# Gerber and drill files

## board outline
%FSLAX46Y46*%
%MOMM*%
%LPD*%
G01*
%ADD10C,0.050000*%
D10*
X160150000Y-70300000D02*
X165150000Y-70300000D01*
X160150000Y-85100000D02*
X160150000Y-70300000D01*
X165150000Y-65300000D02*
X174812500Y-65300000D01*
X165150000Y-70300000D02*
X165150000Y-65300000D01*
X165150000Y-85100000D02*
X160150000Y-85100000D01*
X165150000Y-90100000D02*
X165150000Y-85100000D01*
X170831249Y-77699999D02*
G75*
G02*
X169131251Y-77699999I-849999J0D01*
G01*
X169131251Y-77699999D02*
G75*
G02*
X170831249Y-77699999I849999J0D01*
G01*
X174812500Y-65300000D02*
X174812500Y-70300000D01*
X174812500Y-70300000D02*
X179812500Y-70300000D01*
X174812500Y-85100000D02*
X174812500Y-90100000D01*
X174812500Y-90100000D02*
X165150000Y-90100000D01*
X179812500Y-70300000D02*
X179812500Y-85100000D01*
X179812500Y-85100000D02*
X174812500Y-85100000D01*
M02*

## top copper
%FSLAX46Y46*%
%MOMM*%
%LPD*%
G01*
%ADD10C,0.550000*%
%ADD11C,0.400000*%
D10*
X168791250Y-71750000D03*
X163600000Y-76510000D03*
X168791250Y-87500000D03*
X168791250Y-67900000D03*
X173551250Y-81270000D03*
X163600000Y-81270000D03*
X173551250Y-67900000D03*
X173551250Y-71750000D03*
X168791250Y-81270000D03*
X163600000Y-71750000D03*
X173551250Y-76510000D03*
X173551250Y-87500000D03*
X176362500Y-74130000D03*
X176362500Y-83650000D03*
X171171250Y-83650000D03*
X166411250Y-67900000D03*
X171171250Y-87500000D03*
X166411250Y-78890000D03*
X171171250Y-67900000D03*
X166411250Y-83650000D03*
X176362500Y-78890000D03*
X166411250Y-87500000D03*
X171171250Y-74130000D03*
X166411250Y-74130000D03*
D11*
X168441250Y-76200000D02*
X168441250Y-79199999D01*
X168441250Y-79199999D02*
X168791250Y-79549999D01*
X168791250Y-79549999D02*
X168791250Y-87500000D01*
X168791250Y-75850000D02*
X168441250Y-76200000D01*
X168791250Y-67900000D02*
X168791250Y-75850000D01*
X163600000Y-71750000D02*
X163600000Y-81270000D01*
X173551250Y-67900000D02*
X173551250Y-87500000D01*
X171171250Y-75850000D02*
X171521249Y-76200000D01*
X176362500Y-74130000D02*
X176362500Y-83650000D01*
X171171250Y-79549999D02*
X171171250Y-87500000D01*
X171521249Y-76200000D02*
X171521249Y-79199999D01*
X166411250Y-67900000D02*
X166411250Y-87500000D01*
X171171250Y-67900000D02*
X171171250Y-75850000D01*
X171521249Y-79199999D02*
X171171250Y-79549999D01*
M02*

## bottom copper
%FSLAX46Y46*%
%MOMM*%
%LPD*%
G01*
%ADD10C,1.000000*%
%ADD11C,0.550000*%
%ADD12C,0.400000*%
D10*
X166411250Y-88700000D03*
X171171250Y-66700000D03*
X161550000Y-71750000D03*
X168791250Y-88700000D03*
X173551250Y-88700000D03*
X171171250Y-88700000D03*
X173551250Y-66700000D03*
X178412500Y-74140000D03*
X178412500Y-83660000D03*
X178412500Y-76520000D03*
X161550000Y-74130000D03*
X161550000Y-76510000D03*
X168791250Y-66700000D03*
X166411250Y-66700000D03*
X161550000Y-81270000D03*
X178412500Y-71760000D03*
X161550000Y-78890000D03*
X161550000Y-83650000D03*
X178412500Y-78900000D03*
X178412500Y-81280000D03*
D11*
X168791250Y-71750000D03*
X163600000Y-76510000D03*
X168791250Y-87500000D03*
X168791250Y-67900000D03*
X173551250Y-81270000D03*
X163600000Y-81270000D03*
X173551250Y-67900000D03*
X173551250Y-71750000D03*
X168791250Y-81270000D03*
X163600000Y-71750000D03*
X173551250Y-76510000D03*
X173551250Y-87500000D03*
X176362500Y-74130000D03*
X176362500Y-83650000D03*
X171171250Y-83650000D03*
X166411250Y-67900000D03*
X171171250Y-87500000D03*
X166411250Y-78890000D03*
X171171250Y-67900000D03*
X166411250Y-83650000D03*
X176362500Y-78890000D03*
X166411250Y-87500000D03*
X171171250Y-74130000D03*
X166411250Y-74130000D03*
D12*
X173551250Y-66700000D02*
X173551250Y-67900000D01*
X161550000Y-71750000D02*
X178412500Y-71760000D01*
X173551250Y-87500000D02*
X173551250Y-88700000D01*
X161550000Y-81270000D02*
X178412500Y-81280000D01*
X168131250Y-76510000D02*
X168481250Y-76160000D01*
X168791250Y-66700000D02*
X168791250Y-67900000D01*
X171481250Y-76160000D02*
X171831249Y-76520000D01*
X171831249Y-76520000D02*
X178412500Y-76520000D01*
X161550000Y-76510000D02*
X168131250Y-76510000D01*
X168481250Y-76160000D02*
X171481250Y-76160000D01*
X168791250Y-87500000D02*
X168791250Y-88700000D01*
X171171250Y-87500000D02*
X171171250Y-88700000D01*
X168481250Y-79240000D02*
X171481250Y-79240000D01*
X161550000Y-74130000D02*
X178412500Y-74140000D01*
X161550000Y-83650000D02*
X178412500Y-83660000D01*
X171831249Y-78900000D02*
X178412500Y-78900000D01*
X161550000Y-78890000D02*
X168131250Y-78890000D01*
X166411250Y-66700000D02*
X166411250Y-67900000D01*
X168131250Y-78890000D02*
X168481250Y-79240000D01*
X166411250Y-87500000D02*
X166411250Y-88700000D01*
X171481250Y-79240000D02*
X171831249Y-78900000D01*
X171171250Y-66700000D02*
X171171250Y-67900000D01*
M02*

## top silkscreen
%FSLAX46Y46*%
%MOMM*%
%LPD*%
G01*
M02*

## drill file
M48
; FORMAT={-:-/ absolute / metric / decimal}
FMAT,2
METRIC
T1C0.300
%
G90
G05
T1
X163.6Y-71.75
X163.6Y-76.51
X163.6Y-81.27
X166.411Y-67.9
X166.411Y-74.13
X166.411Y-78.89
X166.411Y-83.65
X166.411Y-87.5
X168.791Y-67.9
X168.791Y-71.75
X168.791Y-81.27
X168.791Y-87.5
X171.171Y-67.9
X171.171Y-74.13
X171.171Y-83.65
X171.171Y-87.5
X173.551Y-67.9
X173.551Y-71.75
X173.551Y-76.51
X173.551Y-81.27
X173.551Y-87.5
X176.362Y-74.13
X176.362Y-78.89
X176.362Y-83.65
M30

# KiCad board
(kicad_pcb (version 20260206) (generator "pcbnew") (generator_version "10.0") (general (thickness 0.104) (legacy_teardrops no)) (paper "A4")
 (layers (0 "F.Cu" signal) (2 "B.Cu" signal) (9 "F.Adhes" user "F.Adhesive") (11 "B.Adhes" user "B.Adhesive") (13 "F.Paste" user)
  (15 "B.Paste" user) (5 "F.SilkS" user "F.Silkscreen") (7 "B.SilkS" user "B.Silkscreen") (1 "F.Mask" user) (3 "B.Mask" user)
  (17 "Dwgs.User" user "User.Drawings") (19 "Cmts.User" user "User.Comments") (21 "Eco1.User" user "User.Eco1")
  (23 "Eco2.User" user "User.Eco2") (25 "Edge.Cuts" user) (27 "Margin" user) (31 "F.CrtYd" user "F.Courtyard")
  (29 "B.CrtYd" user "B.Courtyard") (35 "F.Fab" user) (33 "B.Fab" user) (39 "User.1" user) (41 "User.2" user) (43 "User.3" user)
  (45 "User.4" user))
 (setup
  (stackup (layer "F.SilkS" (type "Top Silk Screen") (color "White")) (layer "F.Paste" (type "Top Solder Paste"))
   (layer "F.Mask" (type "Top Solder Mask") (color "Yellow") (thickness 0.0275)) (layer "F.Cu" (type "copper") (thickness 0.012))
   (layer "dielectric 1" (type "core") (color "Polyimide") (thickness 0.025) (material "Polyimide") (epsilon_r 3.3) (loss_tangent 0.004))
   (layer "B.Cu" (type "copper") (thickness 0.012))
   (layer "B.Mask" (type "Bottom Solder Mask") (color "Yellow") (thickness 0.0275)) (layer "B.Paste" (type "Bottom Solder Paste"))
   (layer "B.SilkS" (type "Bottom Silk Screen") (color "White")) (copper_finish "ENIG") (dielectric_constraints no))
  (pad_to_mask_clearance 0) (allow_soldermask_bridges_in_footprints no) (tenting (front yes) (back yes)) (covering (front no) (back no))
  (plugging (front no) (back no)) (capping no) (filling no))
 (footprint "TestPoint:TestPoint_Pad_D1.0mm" (layer "B.Cu") (at 166.41125 88.7)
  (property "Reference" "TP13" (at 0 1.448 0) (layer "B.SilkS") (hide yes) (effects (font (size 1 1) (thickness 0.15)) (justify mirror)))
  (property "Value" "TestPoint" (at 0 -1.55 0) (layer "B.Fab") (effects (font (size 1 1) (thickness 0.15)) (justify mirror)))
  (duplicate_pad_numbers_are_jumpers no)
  (pad "1" smd circle (at 0 0) (size 1 1) (layers "B.Cu" "B.Mask") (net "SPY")))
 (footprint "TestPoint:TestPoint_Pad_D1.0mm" (layer "B.Cu") (at 171.17125 66.7 180)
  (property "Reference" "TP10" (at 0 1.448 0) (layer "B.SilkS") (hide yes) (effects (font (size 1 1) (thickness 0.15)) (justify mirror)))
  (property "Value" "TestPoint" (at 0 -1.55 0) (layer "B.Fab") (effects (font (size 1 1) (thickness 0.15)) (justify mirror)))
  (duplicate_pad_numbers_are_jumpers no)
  (pad "1" smd circle (at 0 0 180) (size 1 1) (layers "B.Cu" "B.Mask") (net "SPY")))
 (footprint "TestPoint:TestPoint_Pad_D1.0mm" (layer "B.Cu") (at 161.55 71.75 -90)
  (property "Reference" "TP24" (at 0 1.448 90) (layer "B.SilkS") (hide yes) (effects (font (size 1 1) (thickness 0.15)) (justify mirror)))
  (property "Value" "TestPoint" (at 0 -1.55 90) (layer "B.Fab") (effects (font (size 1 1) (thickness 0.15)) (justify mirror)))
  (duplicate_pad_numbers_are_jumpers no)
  (pad "1" smd circle (at 0 0 270) (size 1 1) (layers "B.Cu" "B.Mask") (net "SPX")))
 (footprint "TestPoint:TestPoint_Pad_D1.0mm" (layer "B.Cu") (at 168.79125 88.7)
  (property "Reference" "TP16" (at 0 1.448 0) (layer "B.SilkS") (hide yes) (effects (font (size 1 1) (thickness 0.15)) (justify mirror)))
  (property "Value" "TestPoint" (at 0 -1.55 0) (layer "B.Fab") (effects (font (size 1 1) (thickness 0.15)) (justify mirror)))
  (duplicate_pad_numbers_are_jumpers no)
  (pad "1" smd circle (at 0 0) (size 1 1) (layers "B.Cu" "B.Mask") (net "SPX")))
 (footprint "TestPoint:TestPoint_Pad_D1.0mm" (layer "B.Cu") (at 173.55125 88.7)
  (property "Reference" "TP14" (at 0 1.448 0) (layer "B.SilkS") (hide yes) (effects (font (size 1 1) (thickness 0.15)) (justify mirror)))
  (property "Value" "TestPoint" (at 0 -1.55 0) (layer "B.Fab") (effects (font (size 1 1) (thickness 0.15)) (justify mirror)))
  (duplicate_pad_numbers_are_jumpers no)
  (pad "1" smd circle (at 0 0) (size 1 1) (layers "B.Cu" "B.Mask") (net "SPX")))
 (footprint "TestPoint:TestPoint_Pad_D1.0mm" (layer "B.Cu") (at 171.17125 88.7)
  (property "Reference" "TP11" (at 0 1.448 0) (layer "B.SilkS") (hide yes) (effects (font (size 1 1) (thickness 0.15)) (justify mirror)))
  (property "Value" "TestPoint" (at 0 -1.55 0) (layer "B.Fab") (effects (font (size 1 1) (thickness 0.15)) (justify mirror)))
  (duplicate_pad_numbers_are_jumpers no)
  (pad "1" smd circle (at 0 0) (size 1 1) (layers "B.Cu" "B.Mask") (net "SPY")))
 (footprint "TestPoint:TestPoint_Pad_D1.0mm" (layer "B.Cu") (at 173.55125 66.7 180)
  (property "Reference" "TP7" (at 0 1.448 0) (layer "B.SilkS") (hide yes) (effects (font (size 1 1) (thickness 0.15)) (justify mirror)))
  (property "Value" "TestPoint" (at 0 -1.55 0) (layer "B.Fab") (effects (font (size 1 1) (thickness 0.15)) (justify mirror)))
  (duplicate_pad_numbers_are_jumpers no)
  (pad "1" smd circle (at 0 0 180) (size 1 1) (layers "B.Cu" "B.Mask") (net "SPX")))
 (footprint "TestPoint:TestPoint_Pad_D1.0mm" (layer "B.Cu") (at 178.4125 74.14 90)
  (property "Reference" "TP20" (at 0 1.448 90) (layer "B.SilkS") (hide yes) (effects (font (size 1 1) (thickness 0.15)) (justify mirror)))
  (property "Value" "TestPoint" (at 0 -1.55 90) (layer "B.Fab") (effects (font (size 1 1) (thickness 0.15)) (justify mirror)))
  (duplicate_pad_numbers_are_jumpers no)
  (pad "1" smd circle (at 0 0 90) (size 1 1) (layers "B.Cu" "B.Mask") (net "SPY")))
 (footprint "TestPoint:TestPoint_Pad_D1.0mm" (layer "B.Cu") (at 178.4125 83.66 90)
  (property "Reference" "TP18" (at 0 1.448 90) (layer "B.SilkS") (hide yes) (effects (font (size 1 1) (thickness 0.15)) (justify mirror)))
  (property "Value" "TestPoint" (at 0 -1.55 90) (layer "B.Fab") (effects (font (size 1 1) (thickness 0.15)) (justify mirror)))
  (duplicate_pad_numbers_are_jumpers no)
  (pad "1" smd circle (at 0 0 90) (size 1 1) (layers "B.Cu" "B.Mask") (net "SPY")))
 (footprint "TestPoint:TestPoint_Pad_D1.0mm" (layer "B.Cu") (at 178.4125 76.52 90)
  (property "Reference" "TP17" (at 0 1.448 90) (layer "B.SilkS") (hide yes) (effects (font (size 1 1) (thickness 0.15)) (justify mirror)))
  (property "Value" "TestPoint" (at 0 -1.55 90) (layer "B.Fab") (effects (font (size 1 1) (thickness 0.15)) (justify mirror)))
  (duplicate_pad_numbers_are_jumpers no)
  (pad "1" smd circle (at 0 0 90) (size 1 1) (layers "B.Cu" "B.Mask") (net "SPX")))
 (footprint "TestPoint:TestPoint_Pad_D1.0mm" (layer "B.Cu") (at 161.55 74.13 -90)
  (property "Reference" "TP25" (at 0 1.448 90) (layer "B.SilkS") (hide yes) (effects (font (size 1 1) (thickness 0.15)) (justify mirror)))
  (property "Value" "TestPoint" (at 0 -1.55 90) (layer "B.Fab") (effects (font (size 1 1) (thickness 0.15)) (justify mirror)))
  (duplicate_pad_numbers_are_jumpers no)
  (pad "1" smd circle (at 0 0 270) (size 1 1) (layers "B.Cu" "B.Mask") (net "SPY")))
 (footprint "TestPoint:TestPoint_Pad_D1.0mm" (layer "B.Cu") (at 161.55 76.51 -90)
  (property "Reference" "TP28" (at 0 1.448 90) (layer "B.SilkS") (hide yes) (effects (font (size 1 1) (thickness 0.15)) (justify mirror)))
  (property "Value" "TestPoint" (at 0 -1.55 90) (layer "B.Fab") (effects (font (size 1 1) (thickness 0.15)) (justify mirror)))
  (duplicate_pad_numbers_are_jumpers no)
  (pad "1" smd circle (at 0 0 270) (size 1 1) (layers "B.Cu" "B.Mask") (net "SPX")))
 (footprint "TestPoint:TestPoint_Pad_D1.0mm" (layer "B.Cu") (at 168.79125 66.7 180)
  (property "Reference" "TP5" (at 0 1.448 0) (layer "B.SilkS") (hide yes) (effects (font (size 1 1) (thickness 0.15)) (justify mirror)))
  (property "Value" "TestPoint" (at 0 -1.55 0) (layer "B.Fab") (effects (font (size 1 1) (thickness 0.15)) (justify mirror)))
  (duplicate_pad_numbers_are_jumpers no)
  (pad "1" smd circle (at 0 0 180) (size 1 1) (layers "B.Cu" "B.Mask") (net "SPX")))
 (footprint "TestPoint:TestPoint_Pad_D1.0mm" (layer "B.Cu") (at 166.41125 66.7 180)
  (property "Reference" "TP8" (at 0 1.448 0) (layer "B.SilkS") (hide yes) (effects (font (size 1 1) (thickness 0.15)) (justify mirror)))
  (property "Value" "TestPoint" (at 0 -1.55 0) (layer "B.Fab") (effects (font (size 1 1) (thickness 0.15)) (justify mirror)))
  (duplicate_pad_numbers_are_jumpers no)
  (pad "1" smd circle (at 0 0 180) (size 1 1) (layers "B.Cu" "B.Mask") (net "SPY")))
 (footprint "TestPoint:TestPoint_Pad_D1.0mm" (layer "B.Cu") (at 161.55 81.27 -90)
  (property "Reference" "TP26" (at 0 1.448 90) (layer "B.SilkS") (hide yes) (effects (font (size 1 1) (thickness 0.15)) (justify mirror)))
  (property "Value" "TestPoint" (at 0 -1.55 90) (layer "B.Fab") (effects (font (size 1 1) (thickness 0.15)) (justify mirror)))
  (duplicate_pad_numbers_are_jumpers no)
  (pad "1" smd circle (at 0 0 270) (size 1 1) (layers "B.Cu" "B.Mask") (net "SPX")))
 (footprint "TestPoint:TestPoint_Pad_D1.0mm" (layer "B.Cu") (at 178.4125 71.76 90)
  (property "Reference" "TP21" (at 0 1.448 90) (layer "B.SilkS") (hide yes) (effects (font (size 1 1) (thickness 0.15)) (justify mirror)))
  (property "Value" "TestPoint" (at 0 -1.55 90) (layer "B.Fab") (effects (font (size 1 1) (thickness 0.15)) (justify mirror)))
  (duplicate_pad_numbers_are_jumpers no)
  (pad "1" smd circle (at 0 0 90) (size 1 1) (layers "B.Cu" "B.Mask") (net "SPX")))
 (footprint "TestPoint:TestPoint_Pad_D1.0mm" (layer "B.Cu") (at 161.55 78.89 -90)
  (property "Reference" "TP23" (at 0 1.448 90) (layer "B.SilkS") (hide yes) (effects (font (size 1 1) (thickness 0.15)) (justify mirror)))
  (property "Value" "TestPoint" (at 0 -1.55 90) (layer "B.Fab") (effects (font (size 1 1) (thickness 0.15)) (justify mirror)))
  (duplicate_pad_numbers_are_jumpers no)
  (pad "1" smd circle (at 0 0 270) (size 1 1) (layers "B.Cu" "B.Mask") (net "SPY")))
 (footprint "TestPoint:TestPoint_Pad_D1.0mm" (layer "B.Cu") (at 161.55 83.65 -90)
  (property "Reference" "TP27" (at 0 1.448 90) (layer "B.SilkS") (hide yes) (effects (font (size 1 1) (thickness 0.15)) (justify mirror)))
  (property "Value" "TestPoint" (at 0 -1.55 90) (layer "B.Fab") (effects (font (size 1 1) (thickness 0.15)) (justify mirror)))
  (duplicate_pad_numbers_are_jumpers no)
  (pad "1" smd circle (at 0 0 270) (size 1 1) (layers "B.Cu" "B.Mask") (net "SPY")))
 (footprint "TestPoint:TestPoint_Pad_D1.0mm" (layer "B.Cu") (at 178.4125 78.9 90)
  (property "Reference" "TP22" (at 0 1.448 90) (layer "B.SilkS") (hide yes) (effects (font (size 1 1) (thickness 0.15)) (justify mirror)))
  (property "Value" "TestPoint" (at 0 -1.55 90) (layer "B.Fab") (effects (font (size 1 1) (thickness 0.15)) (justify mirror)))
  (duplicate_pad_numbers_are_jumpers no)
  (pad "1" smd circle (at 0 0 90) (size 1 1) (layers "B.Cu" "B.Mask") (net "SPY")))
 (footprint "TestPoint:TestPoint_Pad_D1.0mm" (layer "B.Cu") (at 178.4125 81.28 90)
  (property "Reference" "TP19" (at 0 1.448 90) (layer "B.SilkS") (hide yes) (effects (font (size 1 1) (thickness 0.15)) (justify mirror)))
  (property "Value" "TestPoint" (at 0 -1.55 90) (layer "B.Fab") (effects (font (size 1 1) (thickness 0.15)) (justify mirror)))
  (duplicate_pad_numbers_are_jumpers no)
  (pad "1" smd circle (at 0 0 90) (size 1 1) (layers "B.Cu" "B.Mask") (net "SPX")))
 (gr_line (start 160.15 70.3) (end 165.15 70.3) (stroke (width 0.05) (type default)) (layer "Edge.Cuts"))
 (gr_line (start 160.15 85.1) (end 160.15 70.3) (stroke (width 0.05) (type default)) (layer "Edge.Cuts"))
 (gr_line (start 165.15 65.3) (end 174.8125 65.3) (stroke (width 0.05) (type default)) (layer "Edge.Cuts"))
 (gr_line (start 165.15 70.3) (end 165.15 65.3) (stroke (width 0.05) (type default)) (layer "Edge.Cuts"))
 (gr_line (start 165.15 85.1) (end 160.15 85.1) (stroke (width 0.05) (type default)) (layer "Edge.Cuts"))
 (gr_line (start 165.15 90.1) (end 165.15 85.1) (stroke (width 0.05) (type default)) (layer "Edge.Cuts"))
 (gr_circle (center 169.98125 77.699999) (end 170.831249 77.699999) (stroke (width 0.05) (type default)) (fill no) (layer "Edge.Cuts"))
 (gr_line (start 174.8125 65.3) (end 174.8125 70.3) (stroke (width 0.05) (type default)) (layer "Edge.Cuts"))
 (gr_line (start 174.8125 70.3) (end 179.8125 70.3) (stroke (width 0.05) (type default)) (layer "Edge.Cuts"))
 (gr_line (start 174.8125 85.1) (end 174.8125 90.1) (stroke (width 0.05) (type default)) (layer "Edge.Cuts"))
 (gr_line (start 174.8125 90.1) (end 165.15 90.1) (stroke (width 0.05) (type default)) (layer "Edge.Cuts"))
 (gr_line (start 179.8125 70.3) (end 179.8125 85.1) (stroke (width 0.05) (type default)) (layer "Edge.Cuts"))
 (gr_line (start 179.8125 85.1) (end 174.8125 85.1) (stroke (width 0.05) (type default)) (layer "Edge.Cuts"))
 (segment (start 168.44125 76.2) (end 168.44125 79.199999) (width 0.4) (layer "F.Cu") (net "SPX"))
 (segment (start 168.44125 79.199999) (end 168.79125 79.549999) (width 0.4) (layer "F.Cu") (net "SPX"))
 (segment (start 168.79125 79.549999) (end 168.79125 87.5) (width 0.4) (layer "F.Cu") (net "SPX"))
 (segment (start 168.79125 75.85) (end 168.44125 76.2) (width 0.4) (layer "F.Cu") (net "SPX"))
 (segment (start 168.79125 67.9) (end 168.79125 75.85) (width 0.4) (layer "F.Cu") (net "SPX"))
 (segment (start 163.6 71.75) (end 163.6 81.27) (width 0.4) (layer "F.Cu") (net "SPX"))
 (segment (start 173.55125 67.9) (end 173.55125 87.5) (width 0.4) (layer "F.Cu") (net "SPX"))
 (via (at 168.79125 71.75) (size 0.55) (drill 0.3) (layers "F.Cu" "B.Cu") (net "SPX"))
 (via (at 163.6 76.51) (size 0.55) (drill 0.3) (layers "F.Cu" "B.Cu") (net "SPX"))
 (via (at 168.79125 87.5) (size 0.55) (drill 0.3) (layers "F.Cu" "B.Cu") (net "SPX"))
 (via (at 168.79125 67.9) (size 0.55) (drill 0.3) (layers "F.Cu" "B.Cu") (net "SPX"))
 (via (at 173.55125 81.27) (size 0.55) (drill 0.3) (layers "F.Cu" "B.Cu") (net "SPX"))
 (via (at 163.6 81.27) (size 0.55) (drill 0.3) (layers "F.Cu" "B.Cu") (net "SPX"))
 (via (at 173.55125 67.9) (size 0.55) (drill 0.3) (layers "F.Cu" "B.Cu") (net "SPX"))
 (via (at 173.55125 71.75) (size 0.55) (drill 0.3) (layers "F.Cu" "B.Cu") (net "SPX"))
 (via (at 168.79125 81.27) (size 0.55) (drill 0.3) (layers "F.Cu" "B.Cu") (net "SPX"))
 (via (at 163.6 71.75) (size 0.55) (drill 0.3) (layers "F.Cu" "B.Cu") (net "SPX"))
 (via (at 173.55125 76.51) (size 0.55) (drill 0.3) (layers "F.Cu" "B.Cu") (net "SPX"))
 (via (at 173.55125 87.5) (size 0.55) (drill 0.3) (layers "F.Cu" "B.Cu") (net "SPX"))
 (segment (start 173.55125 66.7) (end 173.55125 67.9) (width 0.4) (layer "B.Cu") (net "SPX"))
 (segment (start 161.55 71.75) (end 178.4125 71.76) (width 0.4) (layer "B.Cu") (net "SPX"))
 (segment (start 173.55125 87.5) (end 173.55125 88.7) (width 0.4) (layer "B.Cu") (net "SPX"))
 (segment (start 161.55 81.27) (end 178.4125 81.28) (width 0.4) (layer "B.Cu") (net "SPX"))
 (segment (start 168.13125 76.51) (end 168.48125 76.16) (width 0.4) (layer "B.Cu") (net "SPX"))
 (segment (start 168.79125 66.7) (end 168.79125 67.9) (width 0.4) (layer "B.Cu") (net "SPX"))
 (segment (start 171.48125 76.16) (end 171.831249 76.52) (width 0.4) (layer "B.Cu") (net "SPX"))
 (segment (start 171.831249 76.52) (end 178.4125 76.52) (width 0.4) (layer "B.Cu") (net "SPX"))
 (segment (start 161.55 76.51) (end 168.13125 76.51) (width 0.4) (layer "B.Cu") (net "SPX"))
 (segment (start 168.48125 76.16) (end 171.48125 76.16) (width 0.4) (layer "B.Cu") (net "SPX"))
 (segment (start 168.79125 87.5) (end 168.79125 88.7) (width 0.4) (layer "B.Cu") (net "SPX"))
 (segment (start 171.17125 75.85) (end 171.521249 76.2) (width 0.4) (layer "F.Cu") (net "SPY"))
 (segment (start 176.3625 74.13) (end 176.3625 83.65) (width 0.4) (layer "F.Cu") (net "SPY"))
 (segment (start 171.17125 79.549999) (end 171.17125 87.5) (width 0.4) (layer "F.Cu") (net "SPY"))
 (segment (start 171.521249 76.2) (end 171.521249 79.199999) (width 0.4) (layer "F.Cu") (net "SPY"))
 (segment (start 166.41125 67.9) (end 166.41125 87.5) (width 0.4) (layer "F.Cu") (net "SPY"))
 (segment (start 171.17125 67.9) (end 171.17125 75.85) (width 0.4) (layer "F.Cu") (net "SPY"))
 (segment (start 171.521249 79.199999) (end 171.17125 79.549999) (width 0.4) (layer "F.Cu") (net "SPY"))
 (via (at 176.3625 74.13) (size 0.55) (drill 0.3) (layers "F.Cu" "B.Cu") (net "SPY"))
 (via (at 176.3625 83.65) (size 0.55) (drill 0.3) (layers "F.Cu" "B.Cu") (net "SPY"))
 (via (at 171.17125 83.65) (size 0.55) (drill 0.3) (layers "F.Cu" "B.Cu") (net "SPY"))
 (via (at 166.41125 67.9) (size 0.55) (drill 0.3) (layers "F.Cu" "B.Cu") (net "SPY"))
 (via (at 171.17125 87.5) (size 0.55) (drill 0.3) (layers "F.Cu" "B.Cu") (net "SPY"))
 (via (at 166.41125 78.89) (size 0.55) (drill 0.3) (layers "F.Cu" "B.Cu") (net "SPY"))
 (via (at 171.17125 67.9) (size 0.55) (drill 0.3) (layers "F.Cu" "B.Cu") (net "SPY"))
 (via (at 166.41125 83.65) (size 0.55) (drill 0.3) (layers "F.Cu" "B.Cu") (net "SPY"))
 (via (at 176.3625 78.89) (size 0.55) (drill 0.3) (layers "F.Cu" "B.Cu") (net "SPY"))
 (via (at 166.41125 87.5) (size 0.55) (drill 0.3) (layers "F.Cu" "B.Cu") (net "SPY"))
 (via (at 171.17125 74.13) (size 0.55) (drill 0.3) (layers "F.Cu" "B.Cu") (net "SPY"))
 (via (at 166.41125 74.13) (size 0.55) (drill 0.3) (layers "F.Cu" "B.Cu") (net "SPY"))
 (segment (start 171.17125 87.5) (end 171.17125 88.7) (width 0.4) (layer "B.Cu") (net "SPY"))
 (segment (start 168.48125 79.24) (end 171.48125 79.24) (width 0.4) (layer "B.Cu") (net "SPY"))
 (segment (start 161.55 74.13) (end 178.4125 74.14) (width 0.4) (layer "B.Cu") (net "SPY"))
 (segment (start 161.55 83.65) (end 178.4125 83.66) (width 0.4) (layer "B.Cu") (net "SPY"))
 (segment (start 171.831249 78.9) (end 178.4125 78.9) (width 0.4) (layer "B.Cu") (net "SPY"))
 (segment (start 161.55 78.89) (end 168.13125 78.89) (width 0.4) (layer "B.Cu") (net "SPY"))
 (segment (start 166.41125 66.7) (end 166.41125 67.9) (width 0.4) (layer "B.Cu") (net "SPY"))
 (segment (start 168.13125 78.89) (end 168.48125 79.24) (width 0.4) (layer "B.Cu") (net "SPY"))
 (segment (start 166.41125 87.5) (end 166.41125 88.7) (width 0.4) (layer "B.Cu") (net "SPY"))
 (segment (start 171.48125 79.24) (end 171.831249 78.9) (width 0.4) (layer "B.Cu") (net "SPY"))
 (segment (start 171.17125 66.7) (end 171.17125 67.9) (width 0.4) (layer "B.Cu") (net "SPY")))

